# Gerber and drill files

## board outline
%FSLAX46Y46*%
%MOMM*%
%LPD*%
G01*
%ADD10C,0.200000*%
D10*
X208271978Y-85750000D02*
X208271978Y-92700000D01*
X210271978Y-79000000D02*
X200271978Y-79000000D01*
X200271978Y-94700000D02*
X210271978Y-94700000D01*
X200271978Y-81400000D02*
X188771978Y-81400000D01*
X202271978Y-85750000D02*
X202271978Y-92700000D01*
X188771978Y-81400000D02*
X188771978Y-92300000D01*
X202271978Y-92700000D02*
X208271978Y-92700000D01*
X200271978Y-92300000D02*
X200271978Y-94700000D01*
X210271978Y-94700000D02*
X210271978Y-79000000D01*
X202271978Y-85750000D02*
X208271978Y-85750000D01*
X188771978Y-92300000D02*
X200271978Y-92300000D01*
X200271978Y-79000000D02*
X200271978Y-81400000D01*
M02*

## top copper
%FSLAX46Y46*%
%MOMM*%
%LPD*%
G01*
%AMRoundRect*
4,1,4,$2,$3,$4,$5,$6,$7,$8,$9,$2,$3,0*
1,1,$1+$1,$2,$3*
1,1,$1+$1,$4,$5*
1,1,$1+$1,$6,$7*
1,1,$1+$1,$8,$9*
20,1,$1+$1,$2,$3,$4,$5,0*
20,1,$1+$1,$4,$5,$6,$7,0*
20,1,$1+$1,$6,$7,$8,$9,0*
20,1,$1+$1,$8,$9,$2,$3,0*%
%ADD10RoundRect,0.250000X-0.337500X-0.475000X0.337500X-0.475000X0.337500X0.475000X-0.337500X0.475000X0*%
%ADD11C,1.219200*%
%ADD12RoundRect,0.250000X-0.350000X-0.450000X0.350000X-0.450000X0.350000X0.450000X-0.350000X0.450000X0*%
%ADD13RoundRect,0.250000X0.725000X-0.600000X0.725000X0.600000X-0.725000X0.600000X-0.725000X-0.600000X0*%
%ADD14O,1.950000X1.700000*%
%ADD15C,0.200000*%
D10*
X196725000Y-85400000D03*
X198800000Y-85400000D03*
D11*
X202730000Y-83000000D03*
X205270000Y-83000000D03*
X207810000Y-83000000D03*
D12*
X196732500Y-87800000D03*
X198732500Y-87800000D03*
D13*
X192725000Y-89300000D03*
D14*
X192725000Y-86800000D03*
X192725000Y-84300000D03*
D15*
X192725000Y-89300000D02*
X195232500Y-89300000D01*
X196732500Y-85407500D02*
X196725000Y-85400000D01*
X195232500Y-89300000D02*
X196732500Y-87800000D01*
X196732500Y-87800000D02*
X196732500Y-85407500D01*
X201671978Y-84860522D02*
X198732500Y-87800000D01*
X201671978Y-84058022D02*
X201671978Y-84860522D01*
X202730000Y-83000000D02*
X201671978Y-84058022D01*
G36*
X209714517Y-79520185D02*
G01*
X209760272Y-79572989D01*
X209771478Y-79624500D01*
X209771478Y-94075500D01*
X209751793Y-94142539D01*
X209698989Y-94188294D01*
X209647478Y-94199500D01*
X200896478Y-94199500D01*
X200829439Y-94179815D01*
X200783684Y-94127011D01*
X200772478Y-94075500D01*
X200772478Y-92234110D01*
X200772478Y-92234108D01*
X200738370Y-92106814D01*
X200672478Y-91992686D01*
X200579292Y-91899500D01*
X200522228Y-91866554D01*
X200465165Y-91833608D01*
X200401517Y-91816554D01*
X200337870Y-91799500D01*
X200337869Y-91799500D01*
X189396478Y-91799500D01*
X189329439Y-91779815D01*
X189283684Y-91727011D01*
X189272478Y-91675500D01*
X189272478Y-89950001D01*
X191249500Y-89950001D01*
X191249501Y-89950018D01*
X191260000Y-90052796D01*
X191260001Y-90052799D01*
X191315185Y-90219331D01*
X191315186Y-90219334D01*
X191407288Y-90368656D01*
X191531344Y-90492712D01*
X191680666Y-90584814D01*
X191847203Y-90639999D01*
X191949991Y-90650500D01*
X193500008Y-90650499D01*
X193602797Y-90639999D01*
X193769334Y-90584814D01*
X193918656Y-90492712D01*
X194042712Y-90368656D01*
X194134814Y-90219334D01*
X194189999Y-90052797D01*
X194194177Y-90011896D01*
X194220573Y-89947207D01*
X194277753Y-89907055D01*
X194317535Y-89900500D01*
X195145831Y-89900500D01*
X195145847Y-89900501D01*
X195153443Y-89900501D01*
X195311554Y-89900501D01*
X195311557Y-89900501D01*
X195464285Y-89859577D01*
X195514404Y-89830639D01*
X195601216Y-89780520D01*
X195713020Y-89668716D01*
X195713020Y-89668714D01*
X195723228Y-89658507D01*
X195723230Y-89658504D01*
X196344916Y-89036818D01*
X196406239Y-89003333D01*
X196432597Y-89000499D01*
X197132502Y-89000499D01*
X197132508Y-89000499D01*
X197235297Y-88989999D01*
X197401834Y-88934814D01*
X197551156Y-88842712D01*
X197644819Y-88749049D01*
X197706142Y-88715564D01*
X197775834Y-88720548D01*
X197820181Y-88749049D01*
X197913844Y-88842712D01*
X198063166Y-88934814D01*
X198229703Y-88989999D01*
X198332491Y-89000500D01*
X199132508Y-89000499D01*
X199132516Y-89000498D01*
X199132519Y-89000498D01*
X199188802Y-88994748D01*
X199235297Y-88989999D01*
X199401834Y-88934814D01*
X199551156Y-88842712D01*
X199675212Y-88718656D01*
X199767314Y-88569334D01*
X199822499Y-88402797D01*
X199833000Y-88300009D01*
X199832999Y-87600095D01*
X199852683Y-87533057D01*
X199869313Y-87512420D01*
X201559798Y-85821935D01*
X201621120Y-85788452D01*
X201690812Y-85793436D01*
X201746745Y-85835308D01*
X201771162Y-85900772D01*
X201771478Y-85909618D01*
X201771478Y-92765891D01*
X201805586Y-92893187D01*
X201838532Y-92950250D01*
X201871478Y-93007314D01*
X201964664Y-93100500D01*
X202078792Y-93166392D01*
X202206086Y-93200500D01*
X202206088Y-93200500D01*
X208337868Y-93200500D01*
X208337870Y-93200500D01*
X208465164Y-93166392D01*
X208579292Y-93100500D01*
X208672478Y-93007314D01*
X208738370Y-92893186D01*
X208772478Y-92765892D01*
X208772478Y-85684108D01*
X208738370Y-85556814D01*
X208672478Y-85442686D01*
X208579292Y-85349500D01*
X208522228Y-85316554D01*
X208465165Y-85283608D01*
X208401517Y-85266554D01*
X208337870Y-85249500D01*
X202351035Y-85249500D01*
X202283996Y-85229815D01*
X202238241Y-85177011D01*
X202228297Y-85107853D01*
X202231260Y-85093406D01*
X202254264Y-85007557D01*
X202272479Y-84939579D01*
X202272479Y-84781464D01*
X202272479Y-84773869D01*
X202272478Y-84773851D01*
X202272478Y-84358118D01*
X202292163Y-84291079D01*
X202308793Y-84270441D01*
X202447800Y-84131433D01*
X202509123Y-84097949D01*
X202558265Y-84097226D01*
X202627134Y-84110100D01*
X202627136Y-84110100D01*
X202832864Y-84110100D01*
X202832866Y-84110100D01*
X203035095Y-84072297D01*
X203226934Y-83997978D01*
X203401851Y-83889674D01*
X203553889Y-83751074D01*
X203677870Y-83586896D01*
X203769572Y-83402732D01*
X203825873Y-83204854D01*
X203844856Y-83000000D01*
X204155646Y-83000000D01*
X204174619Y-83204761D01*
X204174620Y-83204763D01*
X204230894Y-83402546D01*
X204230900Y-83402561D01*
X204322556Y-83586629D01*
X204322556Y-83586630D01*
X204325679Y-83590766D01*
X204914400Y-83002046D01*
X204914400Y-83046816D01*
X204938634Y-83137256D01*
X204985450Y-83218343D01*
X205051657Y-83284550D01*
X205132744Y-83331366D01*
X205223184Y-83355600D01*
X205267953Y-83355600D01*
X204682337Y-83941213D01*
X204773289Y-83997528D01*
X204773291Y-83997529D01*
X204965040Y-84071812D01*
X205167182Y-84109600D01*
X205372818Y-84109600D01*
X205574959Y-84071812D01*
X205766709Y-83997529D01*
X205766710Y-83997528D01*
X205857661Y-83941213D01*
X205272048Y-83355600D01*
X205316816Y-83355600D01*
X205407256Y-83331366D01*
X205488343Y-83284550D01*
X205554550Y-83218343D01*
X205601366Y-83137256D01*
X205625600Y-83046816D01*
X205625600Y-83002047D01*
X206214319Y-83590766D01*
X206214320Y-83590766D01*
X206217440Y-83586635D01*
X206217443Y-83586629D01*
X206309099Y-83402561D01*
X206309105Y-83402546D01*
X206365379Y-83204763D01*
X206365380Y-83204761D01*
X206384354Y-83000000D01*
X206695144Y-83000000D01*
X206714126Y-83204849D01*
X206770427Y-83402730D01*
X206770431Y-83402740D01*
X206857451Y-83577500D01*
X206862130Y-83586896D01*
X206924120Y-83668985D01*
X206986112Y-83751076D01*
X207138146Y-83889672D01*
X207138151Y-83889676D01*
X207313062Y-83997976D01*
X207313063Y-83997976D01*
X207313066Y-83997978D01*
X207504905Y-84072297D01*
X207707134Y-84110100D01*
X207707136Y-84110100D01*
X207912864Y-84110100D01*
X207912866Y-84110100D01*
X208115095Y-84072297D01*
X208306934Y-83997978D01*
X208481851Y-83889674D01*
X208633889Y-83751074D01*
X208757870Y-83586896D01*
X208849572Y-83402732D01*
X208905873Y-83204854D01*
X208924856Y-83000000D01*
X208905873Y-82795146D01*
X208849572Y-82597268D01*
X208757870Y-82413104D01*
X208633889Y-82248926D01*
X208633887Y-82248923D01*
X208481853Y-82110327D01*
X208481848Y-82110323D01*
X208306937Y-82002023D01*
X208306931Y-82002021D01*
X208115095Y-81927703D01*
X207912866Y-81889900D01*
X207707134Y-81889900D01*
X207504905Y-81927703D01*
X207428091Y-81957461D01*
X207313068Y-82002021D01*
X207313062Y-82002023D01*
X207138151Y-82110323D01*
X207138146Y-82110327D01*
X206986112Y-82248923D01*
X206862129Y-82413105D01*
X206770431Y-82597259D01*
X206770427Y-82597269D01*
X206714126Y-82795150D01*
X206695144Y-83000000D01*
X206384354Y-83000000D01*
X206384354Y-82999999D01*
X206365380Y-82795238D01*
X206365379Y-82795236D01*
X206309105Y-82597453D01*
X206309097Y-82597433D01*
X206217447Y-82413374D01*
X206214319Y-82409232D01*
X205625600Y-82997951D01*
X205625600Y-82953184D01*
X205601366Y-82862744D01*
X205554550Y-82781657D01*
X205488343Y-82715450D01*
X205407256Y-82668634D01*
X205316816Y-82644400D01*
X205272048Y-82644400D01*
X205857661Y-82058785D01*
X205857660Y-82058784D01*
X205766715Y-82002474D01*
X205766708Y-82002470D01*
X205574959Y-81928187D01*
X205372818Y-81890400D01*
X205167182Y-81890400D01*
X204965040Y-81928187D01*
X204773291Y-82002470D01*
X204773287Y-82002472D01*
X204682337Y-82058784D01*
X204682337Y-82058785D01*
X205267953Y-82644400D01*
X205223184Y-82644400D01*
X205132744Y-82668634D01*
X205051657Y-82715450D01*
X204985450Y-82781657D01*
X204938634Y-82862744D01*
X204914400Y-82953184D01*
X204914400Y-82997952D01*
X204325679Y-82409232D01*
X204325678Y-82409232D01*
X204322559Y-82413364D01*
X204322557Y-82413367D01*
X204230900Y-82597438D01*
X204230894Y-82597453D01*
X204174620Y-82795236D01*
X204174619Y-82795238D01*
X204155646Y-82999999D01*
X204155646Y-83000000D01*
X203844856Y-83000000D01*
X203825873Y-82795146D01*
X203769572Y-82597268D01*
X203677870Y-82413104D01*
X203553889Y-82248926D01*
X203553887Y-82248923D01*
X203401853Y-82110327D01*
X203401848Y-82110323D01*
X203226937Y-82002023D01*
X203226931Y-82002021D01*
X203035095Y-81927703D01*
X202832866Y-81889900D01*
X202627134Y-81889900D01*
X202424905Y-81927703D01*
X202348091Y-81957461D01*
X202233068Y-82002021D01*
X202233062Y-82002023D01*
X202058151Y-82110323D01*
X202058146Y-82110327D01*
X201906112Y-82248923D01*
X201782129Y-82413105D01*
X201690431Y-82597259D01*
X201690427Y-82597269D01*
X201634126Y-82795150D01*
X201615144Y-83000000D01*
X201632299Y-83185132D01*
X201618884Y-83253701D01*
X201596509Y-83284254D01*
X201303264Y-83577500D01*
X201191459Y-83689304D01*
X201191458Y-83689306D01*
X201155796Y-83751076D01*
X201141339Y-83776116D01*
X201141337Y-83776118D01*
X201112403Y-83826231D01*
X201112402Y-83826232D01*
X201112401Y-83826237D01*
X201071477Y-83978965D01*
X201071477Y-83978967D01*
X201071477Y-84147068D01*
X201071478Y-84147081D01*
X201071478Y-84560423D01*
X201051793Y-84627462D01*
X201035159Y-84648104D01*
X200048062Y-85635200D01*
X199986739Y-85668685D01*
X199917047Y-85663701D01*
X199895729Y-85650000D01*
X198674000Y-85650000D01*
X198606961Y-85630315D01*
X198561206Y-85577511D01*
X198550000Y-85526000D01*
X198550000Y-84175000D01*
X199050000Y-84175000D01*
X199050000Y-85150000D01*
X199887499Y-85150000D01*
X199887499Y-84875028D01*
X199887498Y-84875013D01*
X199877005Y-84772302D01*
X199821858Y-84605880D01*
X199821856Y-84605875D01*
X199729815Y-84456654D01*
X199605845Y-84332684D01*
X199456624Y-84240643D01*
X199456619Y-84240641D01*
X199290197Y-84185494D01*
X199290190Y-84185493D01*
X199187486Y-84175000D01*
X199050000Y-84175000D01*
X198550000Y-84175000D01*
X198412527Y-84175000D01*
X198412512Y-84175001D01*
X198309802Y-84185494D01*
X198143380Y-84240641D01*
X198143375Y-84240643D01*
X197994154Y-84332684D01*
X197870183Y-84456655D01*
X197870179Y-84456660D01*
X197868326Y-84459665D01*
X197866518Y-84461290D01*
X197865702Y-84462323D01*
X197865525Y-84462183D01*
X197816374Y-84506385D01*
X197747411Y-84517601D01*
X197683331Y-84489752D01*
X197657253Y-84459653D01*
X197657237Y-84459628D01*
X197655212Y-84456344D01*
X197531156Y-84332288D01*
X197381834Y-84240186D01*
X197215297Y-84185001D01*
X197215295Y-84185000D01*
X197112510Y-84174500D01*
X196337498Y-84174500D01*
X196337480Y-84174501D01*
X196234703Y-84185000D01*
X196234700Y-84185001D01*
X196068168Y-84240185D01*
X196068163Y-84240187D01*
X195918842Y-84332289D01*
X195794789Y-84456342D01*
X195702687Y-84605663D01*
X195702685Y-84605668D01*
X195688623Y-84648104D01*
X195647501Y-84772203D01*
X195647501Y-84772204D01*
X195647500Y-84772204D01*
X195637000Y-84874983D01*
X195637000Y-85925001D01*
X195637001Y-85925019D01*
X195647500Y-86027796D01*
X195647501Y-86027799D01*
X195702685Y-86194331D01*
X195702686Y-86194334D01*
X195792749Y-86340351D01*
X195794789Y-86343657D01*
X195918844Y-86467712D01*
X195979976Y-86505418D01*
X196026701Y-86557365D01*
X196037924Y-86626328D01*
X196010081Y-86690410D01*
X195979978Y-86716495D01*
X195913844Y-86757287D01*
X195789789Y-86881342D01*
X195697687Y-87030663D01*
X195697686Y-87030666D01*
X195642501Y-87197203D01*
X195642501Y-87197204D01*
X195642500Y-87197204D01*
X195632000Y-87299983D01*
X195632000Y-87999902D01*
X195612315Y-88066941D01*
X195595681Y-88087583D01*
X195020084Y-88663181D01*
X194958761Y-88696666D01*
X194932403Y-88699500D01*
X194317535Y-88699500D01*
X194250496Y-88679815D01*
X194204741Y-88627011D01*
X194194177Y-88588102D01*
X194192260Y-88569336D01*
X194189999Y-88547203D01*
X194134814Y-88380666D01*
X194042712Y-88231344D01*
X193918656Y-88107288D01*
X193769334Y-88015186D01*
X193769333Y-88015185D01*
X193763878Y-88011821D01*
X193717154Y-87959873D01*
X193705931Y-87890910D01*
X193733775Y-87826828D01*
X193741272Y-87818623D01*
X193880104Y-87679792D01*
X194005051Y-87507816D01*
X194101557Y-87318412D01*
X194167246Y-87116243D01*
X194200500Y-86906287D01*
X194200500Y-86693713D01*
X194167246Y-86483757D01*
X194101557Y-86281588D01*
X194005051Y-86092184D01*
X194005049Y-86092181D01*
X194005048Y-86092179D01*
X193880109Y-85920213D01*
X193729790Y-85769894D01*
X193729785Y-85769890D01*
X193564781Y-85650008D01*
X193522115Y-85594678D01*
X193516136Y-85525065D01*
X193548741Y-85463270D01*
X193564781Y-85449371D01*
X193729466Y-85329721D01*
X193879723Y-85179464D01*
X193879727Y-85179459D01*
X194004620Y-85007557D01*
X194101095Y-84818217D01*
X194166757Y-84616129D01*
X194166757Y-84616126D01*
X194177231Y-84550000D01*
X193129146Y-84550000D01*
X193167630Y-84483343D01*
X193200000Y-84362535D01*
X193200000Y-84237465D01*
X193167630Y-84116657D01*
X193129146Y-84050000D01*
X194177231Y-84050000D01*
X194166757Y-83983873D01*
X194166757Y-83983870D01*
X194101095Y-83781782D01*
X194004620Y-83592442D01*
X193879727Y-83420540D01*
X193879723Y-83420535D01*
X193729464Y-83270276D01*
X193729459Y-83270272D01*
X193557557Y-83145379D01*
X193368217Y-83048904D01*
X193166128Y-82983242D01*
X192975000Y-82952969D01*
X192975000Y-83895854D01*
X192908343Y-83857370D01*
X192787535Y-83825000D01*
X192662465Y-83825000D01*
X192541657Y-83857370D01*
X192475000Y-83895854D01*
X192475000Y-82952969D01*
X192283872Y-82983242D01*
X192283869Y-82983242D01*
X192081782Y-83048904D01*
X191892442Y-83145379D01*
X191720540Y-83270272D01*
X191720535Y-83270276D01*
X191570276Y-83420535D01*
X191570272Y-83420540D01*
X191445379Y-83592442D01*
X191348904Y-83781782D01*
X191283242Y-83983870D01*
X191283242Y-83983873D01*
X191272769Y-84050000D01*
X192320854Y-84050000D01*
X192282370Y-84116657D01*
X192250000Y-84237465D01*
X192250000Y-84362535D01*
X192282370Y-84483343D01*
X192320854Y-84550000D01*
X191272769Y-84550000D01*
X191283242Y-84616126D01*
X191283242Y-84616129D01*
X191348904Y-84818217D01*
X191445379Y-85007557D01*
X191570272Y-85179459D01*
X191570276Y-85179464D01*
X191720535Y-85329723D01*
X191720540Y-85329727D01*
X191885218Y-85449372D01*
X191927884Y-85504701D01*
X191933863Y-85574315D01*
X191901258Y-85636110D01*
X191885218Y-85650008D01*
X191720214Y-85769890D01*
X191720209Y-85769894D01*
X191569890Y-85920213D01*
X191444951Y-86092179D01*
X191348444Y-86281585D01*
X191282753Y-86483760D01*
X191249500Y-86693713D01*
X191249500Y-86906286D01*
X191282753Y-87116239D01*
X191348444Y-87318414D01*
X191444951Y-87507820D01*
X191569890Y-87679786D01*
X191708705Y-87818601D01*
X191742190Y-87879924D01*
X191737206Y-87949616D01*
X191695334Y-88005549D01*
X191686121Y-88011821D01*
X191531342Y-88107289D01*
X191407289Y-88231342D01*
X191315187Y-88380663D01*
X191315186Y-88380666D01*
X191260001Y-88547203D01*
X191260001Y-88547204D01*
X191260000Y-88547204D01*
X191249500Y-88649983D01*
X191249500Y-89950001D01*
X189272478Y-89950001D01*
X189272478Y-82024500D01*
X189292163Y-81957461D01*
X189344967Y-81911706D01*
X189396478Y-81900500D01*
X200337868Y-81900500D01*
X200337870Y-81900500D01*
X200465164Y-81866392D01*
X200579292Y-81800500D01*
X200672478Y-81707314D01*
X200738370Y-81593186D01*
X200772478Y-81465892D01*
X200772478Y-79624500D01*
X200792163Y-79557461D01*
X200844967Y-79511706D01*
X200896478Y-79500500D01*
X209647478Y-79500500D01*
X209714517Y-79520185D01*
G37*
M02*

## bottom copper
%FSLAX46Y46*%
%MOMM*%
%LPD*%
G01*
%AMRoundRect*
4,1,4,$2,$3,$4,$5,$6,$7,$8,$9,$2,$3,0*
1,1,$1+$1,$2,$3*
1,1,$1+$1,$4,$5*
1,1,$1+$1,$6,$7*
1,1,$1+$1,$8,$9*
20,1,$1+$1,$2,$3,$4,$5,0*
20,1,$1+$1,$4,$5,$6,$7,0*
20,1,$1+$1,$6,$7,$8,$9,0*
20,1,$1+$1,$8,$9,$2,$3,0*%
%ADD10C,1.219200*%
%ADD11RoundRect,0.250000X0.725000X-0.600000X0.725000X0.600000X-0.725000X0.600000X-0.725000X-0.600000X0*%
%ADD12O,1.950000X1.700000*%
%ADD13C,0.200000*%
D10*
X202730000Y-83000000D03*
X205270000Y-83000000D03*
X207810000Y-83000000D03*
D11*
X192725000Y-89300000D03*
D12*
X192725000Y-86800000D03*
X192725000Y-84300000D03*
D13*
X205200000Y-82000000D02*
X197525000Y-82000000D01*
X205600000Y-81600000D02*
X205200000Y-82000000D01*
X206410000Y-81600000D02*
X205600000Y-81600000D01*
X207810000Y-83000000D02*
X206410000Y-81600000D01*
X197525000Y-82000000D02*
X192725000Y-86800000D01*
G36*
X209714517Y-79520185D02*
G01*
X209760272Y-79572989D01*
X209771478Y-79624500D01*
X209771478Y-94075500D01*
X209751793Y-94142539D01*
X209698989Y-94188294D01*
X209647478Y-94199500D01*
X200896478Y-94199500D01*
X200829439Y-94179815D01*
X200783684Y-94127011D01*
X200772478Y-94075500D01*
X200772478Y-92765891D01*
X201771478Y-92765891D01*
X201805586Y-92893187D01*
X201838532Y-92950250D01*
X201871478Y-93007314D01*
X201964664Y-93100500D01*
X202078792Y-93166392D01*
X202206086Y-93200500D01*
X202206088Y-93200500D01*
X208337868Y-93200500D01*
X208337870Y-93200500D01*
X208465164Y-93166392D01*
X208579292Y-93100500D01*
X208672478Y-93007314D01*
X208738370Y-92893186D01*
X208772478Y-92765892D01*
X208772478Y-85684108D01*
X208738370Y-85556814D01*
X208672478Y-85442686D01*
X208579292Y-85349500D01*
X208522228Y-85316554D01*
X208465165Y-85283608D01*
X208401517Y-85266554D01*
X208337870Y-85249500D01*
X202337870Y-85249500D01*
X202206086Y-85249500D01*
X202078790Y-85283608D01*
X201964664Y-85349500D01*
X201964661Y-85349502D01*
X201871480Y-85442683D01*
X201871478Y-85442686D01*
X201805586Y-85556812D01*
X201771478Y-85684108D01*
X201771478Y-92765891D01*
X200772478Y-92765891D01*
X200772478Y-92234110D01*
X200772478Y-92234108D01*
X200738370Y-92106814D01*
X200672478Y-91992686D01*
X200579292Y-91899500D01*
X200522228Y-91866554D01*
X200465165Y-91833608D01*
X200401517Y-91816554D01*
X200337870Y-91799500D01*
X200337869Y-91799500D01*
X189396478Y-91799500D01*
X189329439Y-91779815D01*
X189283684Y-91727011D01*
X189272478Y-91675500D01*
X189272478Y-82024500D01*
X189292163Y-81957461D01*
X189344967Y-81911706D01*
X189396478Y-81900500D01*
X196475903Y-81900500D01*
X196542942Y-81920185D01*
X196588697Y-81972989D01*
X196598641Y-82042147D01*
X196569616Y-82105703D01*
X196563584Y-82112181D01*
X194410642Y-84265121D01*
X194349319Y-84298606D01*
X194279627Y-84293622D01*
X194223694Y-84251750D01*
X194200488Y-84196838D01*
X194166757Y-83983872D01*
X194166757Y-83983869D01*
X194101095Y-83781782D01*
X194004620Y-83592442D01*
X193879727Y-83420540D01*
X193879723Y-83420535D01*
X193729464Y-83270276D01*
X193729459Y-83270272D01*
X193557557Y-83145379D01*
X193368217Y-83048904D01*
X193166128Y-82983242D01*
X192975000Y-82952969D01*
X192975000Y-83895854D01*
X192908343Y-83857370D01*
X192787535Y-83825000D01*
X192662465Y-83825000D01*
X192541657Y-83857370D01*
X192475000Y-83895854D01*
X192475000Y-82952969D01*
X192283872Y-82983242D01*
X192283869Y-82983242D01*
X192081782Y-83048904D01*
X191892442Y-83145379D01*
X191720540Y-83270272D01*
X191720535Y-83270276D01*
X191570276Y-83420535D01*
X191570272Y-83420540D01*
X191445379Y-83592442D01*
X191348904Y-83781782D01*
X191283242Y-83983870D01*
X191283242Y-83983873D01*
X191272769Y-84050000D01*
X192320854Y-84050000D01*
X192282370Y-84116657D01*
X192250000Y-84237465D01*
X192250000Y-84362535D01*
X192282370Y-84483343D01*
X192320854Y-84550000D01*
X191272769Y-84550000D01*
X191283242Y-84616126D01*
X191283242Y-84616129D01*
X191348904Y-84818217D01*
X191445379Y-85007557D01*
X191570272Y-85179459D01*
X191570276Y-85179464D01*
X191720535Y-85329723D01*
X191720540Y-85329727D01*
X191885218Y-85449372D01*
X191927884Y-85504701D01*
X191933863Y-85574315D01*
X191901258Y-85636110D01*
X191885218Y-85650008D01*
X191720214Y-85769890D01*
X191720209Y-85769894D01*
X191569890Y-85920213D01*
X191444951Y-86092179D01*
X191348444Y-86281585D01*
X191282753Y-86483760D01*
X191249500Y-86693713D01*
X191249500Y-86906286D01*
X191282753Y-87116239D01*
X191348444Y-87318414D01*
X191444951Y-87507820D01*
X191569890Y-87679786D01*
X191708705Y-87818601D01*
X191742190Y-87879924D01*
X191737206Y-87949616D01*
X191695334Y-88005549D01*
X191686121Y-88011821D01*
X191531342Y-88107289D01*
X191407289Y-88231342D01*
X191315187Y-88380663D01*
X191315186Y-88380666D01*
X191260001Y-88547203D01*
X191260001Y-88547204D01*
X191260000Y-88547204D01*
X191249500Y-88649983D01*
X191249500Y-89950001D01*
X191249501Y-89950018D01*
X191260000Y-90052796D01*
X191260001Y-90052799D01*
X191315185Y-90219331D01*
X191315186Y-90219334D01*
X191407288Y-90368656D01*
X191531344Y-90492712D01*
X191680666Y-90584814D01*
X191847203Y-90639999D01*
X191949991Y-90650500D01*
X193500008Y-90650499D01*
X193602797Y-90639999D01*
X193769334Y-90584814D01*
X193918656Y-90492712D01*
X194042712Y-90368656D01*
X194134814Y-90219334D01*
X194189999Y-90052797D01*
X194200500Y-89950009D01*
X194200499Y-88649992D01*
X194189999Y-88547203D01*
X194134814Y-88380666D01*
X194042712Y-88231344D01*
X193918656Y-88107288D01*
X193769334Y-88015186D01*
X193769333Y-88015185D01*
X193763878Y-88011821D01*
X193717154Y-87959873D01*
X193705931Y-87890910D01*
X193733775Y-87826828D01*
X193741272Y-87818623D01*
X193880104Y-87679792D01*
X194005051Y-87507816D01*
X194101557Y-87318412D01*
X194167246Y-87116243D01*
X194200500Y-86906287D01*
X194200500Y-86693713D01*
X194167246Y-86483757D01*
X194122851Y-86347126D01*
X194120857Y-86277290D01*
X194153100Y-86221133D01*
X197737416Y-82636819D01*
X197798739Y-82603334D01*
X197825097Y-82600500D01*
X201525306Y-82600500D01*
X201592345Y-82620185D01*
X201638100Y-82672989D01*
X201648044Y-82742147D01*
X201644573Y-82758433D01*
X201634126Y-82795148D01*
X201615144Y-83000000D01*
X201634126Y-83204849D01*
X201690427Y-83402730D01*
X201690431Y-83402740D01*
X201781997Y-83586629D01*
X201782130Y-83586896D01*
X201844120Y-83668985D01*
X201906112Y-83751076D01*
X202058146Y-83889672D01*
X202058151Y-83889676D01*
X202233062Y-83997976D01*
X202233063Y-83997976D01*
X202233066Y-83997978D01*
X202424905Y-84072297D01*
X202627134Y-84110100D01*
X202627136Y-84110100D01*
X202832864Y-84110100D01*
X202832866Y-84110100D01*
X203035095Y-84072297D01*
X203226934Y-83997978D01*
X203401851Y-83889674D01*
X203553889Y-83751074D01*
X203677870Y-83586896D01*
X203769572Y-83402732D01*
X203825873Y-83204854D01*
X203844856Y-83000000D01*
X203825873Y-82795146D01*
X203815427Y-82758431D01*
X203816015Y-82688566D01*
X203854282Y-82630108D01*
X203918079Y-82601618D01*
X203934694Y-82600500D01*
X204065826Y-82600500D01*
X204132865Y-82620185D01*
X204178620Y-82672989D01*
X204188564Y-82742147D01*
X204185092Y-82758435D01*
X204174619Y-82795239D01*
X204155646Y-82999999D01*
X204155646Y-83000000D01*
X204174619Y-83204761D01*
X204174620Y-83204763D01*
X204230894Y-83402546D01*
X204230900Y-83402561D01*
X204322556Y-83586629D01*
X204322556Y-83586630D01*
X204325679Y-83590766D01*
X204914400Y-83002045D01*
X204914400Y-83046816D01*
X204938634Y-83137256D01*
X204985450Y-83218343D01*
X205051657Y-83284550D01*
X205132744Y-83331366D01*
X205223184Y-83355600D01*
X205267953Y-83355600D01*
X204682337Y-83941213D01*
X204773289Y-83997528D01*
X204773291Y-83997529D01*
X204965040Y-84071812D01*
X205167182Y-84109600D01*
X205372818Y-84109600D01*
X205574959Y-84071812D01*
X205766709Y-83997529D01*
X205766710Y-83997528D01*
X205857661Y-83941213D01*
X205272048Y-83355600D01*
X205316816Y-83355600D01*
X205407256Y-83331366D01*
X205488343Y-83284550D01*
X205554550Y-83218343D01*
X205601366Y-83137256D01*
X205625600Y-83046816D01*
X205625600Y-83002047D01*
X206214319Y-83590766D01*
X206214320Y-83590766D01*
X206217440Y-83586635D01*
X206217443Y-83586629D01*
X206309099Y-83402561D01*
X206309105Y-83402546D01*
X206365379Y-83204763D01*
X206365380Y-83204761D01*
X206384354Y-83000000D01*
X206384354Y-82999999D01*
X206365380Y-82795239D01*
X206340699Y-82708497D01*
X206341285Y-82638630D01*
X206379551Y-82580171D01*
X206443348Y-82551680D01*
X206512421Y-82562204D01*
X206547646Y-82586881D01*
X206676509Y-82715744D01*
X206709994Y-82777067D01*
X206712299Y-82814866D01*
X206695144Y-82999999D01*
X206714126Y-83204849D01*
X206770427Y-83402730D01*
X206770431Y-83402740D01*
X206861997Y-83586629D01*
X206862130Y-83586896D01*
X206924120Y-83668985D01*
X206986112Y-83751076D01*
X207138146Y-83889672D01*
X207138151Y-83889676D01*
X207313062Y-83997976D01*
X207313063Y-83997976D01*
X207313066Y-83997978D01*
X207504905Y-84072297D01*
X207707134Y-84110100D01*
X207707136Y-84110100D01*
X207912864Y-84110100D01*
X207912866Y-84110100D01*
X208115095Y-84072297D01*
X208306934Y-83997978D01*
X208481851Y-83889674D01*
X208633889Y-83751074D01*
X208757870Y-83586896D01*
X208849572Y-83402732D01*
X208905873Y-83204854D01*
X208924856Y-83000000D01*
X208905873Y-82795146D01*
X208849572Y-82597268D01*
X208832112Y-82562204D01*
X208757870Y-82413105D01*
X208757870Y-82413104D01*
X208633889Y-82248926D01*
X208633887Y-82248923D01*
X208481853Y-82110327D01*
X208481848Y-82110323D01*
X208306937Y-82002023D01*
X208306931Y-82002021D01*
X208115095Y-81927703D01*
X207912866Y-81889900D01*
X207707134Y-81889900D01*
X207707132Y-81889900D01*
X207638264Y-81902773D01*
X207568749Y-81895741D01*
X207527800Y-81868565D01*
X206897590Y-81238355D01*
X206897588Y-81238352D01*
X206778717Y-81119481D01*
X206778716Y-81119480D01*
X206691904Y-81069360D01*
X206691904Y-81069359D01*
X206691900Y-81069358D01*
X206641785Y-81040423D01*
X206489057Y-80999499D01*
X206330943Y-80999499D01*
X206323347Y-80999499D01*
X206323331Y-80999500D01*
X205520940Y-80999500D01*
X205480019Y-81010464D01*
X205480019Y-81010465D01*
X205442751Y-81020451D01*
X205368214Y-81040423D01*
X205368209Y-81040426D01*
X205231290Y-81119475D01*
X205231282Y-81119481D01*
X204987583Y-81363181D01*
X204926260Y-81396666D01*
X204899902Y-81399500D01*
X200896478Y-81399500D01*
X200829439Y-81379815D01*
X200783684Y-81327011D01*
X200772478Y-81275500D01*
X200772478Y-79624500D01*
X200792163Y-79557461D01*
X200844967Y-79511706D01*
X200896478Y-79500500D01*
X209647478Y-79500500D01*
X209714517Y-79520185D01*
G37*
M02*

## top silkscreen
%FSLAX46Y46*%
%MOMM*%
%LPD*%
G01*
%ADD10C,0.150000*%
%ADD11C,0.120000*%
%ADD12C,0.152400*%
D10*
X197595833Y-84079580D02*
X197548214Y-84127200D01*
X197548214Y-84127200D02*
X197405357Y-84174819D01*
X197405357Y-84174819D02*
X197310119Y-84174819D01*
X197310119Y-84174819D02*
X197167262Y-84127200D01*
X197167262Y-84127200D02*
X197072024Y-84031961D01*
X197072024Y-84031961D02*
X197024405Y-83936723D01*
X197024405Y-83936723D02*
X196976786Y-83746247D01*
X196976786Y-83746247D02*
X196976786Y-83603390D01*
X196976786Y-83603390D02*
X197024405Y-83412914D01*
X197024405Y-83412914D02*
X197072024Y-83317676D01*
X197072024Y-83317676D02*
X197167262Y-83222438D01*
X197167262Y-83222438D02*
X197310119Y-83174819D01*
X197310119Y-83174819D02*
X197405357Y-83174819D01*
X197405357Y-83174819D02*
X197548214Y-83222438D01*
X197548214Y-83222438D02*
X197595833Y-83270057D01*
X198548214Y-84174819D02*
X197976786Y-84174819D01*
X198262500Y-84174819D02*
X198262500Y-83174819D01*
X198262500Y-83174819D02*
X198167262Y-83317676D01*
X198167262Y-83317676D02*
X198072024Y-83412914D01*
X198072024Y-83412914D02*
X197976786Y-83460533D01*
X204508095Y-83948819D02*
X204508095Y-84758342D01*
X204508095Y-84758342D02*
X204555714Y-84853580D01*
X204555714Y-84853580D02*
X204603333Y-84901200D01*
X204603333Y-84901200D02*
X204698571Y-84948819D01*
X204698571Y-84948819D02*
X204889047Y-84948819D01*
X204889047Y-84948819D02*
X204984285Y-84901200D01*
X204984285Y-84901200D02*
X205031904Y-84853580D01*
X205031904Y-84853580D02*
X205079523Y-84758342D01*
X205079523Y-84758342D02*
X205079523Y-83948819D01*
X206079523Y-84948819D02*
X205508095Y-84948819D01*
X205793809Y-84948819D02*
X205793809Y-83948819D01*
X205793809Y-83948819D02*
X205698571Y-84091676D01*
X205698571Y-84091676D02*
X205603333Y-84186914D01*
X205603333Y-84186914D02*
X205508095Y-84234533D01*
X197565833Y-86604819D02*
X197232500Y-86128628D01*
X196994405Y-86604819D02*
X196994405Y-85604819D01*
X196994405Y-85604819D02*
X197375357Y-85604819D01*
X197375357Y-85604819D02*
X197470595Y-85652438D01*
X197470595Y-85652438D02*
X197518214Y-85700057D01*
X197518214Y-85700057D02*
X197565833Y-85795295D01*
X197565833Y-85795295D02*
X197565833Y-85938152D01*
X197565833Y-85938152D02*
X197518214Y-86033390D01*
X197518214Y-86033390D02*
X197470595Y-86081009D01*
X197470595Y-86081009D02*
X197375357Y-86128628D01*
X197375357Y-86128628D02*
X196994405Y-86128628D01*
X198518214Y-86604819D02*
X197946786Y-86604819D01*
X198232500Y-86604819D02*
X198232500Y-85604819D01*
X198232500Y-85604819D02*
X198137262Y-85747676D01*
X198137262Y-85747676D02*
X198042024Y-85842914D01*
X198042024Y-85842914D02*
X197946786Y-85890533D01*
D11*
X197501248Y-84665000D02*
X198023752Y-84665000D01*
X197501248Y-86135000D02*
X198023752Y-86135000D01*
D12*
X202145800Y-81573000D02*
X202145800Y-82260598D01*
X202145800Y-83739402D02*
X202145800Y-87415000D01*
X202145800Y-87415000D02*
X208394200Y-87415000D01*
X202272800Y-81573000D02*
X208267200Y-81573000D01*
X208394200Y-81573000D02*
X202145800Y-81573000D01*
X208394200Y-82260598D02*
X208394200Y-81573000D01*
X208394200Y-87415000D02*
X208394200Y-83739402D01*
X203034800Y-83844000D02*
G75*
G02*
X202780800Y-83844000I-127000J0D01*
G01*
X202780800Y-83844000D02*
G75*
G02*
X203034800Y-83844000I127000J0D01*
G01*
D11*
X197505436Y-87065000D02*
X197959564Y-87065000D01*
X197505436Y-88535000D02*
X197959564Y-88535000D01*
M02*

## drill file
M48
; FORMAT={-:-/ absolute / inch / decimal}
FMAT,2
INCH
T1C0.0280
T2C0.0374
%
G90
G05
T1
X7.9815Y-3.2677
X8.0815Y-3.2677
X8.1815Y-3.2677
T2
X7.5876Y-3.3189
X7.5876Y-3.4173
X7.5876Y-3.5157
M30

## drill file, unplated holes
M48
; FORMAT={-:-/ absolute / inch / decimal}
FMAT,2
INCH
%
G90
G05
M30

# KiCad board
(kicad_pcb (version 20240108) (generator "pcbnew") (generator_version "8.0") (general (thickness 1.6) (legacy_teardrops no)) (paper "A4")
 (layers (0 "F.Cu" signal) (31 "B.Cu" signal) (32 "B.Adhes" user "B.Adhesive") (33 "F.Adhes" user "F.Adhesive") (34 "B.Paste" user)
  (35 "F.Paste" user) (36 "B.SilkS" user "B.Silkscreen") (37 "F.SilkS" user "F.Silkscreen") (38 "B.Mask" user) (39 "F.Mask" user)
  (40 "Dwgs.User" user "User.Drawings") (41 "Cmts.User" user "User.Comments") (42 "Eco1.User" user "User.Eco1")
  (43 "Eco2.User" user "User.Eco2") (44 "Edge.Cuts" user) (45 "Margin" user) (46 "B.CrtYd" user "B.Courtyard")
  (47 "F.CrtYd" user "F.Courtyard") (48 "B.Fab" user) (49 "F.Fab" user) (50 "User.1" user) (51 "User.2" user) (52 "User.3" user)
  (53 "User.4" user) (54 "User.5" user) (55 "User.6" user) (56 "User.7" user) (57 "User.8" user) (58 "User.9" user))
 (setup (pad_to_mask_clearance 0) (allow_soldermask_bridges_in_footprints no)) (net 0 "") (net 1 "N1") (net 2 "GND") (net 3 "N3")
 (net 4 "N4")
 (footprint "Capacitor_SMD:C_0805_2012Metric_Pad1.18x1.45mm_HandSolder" (layer "F.Cu") (at 197.7625 85.4)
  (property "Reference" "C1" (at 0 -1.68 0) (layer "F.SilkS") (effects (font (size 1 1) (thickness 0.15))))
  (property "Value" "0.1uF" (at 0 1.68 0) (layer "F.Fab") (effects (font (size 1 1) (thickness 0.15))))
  (fp_line (start -0.261252 -0.735) (end 0.261252 -0.735) (stroke (width 0.12) (type solid)) (layer "F.SilkS"))
  (fp_line (start -0.261252 0.735) (end 0.261252 0.735) (stroke (width 0.12) (type solid)) (layer "F.SilkS"))
  (pad "1" smd roundrect (at -1.0375 0) (size 1.175 1.45) (layers "F.Cu" "F.Paste" "F.Mask") (roundrect_rratio 0.2127659574) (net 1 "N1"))
  (pad "2" smd roundrect (at 1.0375 0) (size 1.175 1.45) (layers "F.Cu" "F.Paste" "F.Mask") (roundrect_rratio 0.2127659574) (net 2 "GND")))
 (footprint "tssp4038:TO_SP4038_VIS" (layer "F.Cu") (at 205.27 83)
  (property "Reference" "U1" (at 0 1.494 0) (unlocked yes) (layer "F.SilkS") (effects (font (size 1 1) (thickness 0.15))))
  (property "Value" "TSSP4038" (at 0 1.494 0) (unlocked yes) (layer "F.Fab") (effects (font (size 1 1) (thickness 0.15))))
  (fp_line (start -3.1242 -1.427) (end -3.1242 -0.739402) (stroke (width 0.1524) (type solid)) (layer "F.SilkS"))
  (fp_line (start -3.1242 0.739402) (end -3.1242 4.415) (stroke (width 0.1524) (type solid)) (layer "F.SilkS"))
  (fp_line (start -3.1242 4.415) (end 3.1242 4.415) (stroke (width 0.1524) (type solid)) (layer "F.SilkS"))
  (fp_line (start -2.9972 -1.427) (end 2.9972 -1.427) (stroke (width 0.1524) (type solid)) (layer "F.SilkS"))
  (fp_line (start 3.1242 -1.427) (end -3.1242 -1.427) (stroke (width 0.1524) (type solid)) (layer "F.SilkS"))
  (fp_line (start 3.1242 -0.739402) (end 3.1242 -1.427) (stroke (width 0.1524) (type solid)) (layer "F.SilkS"))
  (fp_line (start 3.1242 4.415) (end 3.1242 0.739402) (stroke (width 0.1524) (type solid)) (layer "F.SilkS"))
  (fp_circle (center -2.3622 0.844) (end -2.2352 0.844) (stroke (width 0.1524) (type solid)) (fill none) (layer "F.SilkS"))
  (pad "1" thru_hole circle (at -2.54 0) (size 1.2192 1.2192) (drill 0.7112) (layers "*.Cu" "*.Mask") (remove_unused_layers no) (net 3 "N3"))
  (pad "2" thru_hole circle (at 0 0) (size 1.2192 1.2192) (drill 0.7112) (layers "*.Cu" "*.Mask") (remove_unused_layers no) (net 2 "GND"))
  (pad "3" thru_hole circle (at 2.54 0) (size 1.2192 1.2192) (drill 0.7112) (layers "*.Cu" "*.Mask") (remove_unused_layers no) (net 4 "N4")))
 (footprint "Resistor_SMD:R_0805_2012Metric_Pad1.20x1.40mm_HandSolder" (layer "F.Cu") (at 197.7325 87.8)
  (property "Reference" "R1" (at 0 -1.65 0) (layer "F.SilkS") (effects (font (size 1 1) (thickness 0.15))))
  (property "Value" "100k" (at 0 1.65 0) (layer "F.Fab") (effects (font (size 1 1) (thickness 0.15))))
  (fp_line (start -0.227064 -0.735) (end 0.227064 -0.735) (stroke (width 0.12) (type solid)) (layer "F.SilkS"))
  (fp_line (start -0.227064 0.735) (end 0.227064 0.735) (stroke (width 0.12) (type solid)) (layer "F.SilkS"))
  (pad "1" smd roundrect (at -1 0) (size 1.2 1.4) (layers "F.Cu" "F.Paste" "F.Mask") (roundrect_rratio 0.2083333333) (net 1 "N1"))
  (pad "2" smd roundrect (at 1 0) (size 1.2 1.4) (layers "F.Cu" "F.Paste" "F.Mask") (roundrect_rratio 0.2083333333) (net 3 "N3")))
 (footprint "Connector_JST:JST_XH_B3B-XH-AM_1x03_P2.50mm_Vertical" (layer "B.Cu") (at 192.725 89.3 90)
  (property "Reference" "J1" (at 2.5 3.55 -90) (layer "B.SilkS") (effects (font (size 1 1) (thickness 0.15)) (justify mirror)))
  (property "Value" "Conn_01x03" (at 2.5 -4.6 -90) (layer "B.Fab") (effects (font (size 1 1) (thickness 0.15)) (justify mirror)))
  (pad "1" thru_hole roundrect (at 0 0 90) (size 1.7 1.95) (drill 0.95) (layers "*.Cu" "*.Mask") (remove_unused_layers no)
   (roundrect_rratio 0.1470588235) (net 1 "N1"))
  (pad "2" thru_hole oval (at 2.5 0 90) (size 1.7 1.95) (drill 0.95) (layers "*.Cu" "*.Mask") (remove_unused_layers no) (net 4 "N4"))
  (pad "3" thru_hole oval (at 5 0 90) (size 1.7 1.95) (drill 0.95) (layers "*.Cu" "*.Mask") (remove_unused_layers no) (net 2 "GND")))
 (gr_line (start 208.271978 85.75) (end 208.271978 92.7) (stroke (width 0.2) (type default)) (layer "Edge.Cuts"))
 (gr_line (start 210.271978 79) (end 200.271978 79) (stroke (width 0.2) (type default)) (layer "Edge.Cuts"))
 (gr_line (start 200.271978 94.7) (end 210.271978 94.7) (stroke (width 0.2) (type default)) (layer "Edge.Cuts"))
 (gr_line (start 200.271978 81.4) (end 188.771978 81.4) (stroke (width 0.2) (type default)) (layer "Edge.Cuts"))
 (gr_line (start 202.271978 85.75) (end 202.271978 92.7) (stroke (width 0.2) (type default)) (layer "Edge.Cuts"))
 (gr_line (start 188.771978 81.4) (end 188.771978 92.3) (stroke (width 0.2) (type default)) (layer "Edge.Cuts"))
 (gr_line (start 202.271978 92.7) (end 208.271978 92.7) (stroke (width 0.2) (type default)) (layer "Edge.Cuts"))
 (gr_line (start 200.271978 92.3) (end 200.271978 94.7) (stroke (width 0.2) (type default)) (layer "Edge.Cuts"))
 (gr_line (start 210.271978 94.7) (end 210.271978 79) (stroke (width 0.2) (type default)) (layer "Edge.Cuts"))
 (gr_line (start 202.271978 85.75) (end 208.271978 85.75) (stroke (width 0.2) (type default)) (layer "Edge.Cuts"))
 (gr_line (start 188.771978 92.3) (end 200.271978 92.3) (stroke (width 0.2) (type default)) (layer "Edge.Cuts"))
 (gr_line (start 200.271978 79) (end 200.271978 81.4) (stroke (width 0.2) (type default)) (layer "Edge.Cuts"))
 (segment (start 205.2 82) (end 197.525 82) (width 0.2) (layer "B.Cu") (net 4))
 (segment (start 205.6 81.6) (end 205.2 82) (width 0.2) (layer "B.Cu") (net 4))
 (segment (start 206.41 81.6) (end 205.6 81.6) (width 0.2) (layer "B.Cu") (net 4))
 (segment (start 207.81 83) (end 206.41 81.6) (width 0.2) (layer "B.Cu") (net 4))
 (segment (start 197.525 82) (end 192.725 86.8) (width 0.2) (layer "B.Cu") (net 4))
 (segment (start 192.725 89.3) (end 195.2325 89.3) (width 0.2) (layer "F.Cu") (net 1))
 (segment (start 196.7325 85.4075) (end 196.725 85.4) (width 0.2) (layer "F.Cu") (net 1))
 (segment (start 195.2325 89.3) (end 196.7325 87.8) (width 0.2) (layer "F.Cu") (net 1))
 (segment (start 196.7325 87.8) (end 196.7325 85.4075) (width 0.2) (layer "F.Cu") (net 1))
 (segment (start 201.671978 84.860522) (end 198.7325 87.8) (width 0.2) (layer "F.Cu") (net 3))
 (segment (start 201.671978 84.058022) (end 201.671978 84.860522) (width 0.2) (layer "F.Cu") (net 3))
 (segment (start 202.73 83) (end 201.671978 84.058022) (width 0.2) (layer "F.Cu") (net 3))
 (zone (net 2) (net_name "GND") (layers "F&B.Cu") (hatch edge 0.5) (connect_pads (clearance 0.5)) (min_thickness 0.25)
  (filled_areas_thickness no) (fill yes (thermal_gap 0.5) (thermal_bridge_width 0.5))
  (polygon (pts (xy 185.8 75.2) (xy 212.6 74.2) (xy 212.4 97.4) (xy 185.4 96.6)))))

